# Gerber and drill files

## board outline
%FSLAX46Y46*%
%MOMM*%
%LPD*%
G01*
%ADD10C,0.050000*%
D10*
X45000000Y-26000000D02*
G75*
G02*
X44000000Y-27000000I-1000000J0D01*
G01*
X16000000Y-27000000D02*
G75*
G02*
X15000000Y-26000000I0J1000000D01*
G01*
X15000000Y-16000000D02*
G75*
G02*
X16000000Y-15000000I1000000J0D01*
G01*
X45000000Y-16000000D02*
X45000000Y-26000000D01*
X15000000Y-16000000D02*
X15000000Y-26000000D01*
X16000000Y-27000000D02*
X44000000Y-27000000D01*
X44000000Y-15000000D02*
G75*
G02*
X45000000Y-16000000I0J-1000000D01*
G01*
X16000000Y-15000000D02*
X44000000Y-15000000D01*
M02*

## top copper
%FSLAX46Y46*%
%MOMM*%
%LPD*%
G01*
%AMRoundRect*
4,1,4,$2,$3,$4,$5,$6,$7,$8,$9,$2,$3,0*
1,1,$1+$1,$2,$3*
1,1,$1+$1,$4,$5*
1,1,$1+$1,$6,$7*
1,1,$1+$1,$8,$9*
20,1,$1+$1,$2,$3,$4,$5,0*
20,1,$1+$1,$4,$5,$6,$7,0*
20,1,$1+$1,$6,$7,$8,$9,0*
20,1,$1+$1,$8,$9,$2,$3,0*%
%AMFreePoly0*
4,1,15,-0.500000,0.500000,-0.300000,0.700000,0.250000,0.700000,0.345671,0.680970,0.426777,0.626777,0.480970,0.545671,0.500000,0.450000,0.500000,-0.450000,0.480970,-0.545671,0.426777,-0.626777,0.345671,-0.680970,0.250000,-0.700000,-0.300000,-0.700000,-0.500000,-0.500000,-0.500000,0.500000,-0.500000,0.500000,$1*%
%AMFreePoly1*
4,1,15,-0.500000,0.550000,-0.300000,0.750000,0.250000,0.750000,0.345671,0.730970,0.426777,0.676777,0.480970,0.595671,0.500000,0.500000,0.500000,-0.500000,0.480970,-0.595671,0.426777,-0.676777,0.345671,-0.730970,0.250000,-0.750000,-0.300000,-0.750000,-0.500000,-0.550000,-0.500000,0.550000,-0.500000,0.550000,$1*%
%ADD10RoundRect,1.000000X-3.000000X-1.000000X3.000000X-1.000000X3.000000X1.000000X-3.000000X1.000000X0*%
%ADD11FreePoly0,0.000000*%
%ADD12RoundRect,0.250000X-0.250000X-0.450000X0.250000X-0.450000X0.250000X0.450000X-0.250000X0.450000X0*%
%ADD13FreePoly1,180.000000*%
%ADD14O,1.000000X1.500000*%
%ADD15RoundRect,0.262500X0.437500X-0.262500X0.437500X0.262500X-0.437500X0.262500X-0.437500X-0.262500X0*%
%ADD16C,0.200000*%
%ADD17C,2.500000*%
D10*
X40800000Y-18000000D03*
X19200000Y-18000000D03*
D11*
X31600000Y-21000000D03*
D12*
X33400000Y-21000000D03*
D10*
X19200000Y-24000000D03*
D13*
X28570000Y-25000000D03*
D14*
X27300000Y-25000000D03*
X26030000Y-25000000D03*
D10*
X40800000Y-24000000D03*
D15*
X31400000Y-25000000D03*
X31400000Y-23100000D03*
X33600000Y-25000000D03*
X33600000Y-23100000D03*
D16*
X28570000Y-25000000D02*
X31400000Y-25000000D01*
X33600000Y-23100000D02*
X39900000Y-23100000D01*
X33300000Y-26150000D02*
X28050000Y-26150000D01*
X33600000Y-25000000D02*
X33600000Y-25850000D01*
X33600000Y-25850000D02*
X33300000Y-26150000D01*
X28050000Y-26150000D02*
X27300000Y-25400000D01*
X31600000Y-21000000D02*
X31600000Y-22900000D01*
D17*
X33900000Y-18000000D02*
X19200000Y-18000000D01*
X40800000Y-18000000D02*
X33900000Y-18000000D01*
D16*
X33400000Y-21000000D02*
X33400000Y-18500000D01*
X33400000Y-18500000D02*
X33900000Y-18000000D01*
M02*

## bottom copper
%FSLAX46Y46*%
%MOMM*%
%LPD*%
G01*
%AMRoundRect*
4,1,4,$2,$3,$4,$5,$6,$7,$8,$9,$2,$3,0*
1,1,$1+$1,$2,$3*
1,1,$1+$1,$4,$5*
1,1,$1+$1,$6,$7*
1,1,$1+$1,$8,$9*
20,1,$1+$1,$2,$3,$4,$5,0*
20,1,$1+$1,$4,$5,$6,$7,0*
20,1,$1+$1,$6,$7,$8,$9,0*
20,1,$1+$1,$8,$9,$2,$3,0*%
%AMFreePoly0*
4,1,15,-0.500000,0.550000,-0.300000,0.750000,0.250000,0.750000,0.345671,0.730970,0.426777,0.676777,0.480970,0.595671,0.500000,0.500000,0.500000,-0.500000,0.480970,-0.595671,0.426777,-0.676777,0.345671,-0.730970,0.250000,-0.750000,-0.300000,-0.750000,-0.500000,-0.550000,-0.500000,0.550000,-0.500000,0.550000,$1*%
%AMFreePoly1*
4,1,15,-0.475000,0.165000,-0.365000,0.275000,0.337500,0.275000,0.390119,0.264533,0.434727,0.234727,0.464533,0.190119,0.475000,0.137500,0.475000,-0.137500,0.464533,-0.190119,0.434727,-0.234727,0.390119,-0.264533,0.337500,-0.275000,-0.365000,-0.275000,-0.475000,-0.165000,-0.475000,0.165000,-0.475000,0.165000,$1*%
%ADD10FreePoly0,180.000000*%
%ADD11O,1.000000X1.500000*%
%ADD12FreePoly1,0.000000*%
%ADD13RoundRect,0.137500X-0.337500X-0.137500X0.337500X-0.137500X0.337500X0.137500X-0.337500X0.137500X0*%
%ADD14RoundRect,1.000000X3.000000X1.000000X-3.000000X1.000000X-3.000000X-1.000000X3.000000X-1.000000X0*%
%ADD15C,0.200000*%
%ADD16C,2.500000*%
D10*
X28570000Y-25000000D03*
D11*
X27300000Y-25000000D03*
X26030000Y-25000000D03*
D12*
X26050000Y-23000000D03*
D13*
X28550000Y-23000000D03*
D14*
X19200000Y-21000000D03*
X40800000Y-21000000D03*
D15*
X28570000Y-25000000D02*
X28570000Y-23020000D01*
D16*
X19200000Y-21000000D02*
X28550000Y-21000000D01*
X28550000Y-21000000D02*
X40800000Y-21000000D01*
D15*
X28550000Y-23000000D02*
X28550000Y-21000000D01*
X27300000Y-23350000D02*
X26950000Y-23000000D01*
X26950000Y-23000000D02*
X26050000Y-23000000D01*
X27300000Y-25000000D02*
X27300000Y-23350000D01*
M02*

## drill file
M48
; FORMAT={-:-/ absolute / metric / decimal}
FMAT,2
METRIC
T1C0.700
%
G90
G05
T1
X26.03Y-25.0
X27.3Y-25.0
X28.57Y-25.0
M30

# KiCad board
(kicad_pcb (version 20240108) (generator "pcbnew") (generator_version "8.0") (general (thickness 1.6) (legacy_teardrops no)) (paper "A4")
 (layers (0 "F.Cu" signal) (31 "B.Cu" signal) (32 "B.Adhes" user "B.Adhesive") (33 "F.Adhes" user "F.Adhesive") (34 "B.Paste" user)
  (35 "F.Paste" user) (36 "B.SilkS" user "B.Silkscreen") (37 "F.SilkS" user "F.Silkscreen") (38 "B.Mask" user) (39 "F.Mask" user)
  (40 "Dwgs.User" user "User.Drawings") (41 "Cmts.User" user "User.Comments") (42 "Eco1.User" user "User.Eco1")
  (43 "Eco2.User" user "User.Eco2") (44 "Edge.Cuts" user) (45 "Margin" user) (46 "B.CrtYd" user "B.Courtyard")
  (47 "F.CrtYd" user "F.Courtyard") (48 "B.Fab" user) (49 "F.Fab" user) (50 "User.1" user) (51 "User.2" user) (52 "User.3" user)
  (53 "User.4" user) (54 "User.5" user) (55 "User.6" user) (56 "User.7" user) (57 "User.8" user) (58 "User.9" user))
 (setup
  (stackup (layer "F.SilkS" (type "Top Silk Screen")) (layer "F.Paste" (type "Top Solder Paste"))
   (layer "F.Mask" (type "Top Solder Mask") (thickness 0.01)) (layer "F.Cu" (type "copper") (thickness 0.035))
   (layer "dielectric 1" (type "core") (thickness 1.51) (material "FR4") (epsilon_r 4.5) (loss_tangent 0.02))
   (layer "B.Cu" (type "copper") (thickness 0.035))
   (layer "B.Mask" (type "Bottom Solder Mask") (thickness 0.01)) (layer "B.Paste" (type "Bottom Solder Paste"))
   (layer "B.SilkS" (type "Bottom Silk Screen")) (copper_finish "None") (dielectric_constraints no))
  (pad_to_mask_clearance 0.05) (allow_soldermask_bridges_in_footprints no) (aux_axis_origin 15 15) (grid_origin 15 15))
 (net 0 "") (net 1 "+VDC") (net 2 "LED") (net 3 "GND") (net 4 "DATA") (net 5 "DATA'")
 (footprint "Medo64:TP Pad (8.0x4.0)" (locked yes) (layer "F.Cu") (at 40.8 18)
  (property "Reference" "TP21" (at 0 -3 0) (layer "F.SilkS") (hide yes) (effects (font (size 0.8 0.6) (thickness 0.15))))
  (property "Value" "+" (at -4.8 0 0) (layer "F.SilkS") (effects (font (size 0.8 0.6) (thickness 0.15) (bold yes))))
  (pad "1" smd roundrect (at 0 0) (size 8 4) (layers "F.Cu" "F.Mask") (roundrect_rratio 0.25) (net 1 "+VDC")))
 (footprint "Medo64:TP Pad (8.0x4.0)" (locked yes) (layer "F.Cu") (at 19.2 18)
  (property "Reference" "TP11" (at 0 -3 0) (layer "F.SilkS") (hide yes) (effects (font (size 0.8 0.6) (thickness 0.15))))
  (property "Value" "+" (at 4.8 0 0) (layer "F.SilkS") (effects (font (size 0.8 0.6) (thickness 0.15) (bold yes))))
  (pad "1" smd roundrect (at 0 0) (size 8 4) (layers "F.Cu" "F.Mask") (roundrect_rratio 0.25) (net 1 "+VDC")))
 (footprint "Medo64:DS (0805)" (layer "F.Cu") (at 32.5 21)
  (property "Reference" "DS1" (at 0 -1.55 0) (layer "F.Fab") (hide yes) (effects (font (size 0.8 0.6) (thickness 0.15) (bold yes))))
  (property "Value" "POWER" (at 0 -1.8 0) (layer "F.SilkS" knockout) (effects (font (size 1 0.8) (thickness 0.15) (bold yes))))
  (pad "1" smd roundrect (at -0.9 0) (size 1 1.4) (layers "F.Cu" "F.Paste" "F.Mask") (roundrect_rratio 0.25) (chamfer_ratio 0.2)
   (chamfer top_left bottom_left) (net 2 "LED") (thermal_bridge_angle 45))
  (pad "2" smd roundrect (at 0.9 0) (size 1 1.4) (layers "F.Cu" "F.Paste" "F.Mask") (roundrect_rratio 0.25) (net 1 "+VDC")
   (thermal_bridge_angle 45)))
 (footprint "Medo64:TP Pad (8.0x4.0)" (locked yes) (layer "F.Cu") (at 19.2 24)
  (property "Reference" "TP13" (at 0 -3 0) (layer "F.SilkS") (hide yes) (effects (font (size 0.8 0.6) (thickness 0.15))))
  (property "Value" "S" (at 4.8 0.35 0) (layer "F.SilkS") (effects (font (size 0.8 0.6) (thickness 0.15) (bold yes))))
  (pad "1" smd roundrect (at 0 0) (size 8 4) (layers "F.Cu" "F.Mask") (roundrect_rratio 0.25)))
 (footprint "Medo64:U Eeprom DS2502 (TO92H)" (layer "F.Cu") (at 27.3 25 180)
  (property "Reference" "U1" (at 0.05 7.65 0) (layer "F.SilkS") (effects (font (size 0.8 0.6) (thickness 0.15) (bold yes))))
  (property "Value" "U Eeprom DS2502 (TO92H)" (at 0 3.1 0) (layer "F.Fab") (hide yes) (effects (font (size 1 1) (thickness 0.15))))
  (pad "1" thru_hole roundrect (at -1.27 0 180) (size 1 1.5) (drill 0.7) (layers "*.Cu" "B.Mask") (remove_unused_layers no)
   (roundrect_rratio 0.25) (chamfer_ratio 0.2) (chamfer top_left bottom_left) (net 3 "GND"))
  (pad "2" thru_hole oval (at 0 0 180) (size 1 1.5) (drill 0.7) (layers "*.Cu" "B.Mask") (remove_unused_layers no) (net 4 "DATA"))
  (pad "3" thru_hole oval (at 1.27 0 180) (size 1 1.5) (drill 0.7) (layers "*.Cu" "B.Mask") (remove_unused_layers no)))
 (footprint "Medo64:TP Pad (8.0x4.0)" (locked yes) (layer "F.Cu") (at 40.8 24)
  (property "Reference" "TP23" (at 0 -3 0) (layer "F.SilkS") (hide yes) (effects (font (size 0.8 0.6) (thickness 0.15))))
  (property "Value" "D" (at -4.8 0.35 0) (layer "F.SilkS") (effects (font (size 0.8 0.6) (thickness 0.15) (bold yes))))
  (pad "1" smd roundrect (at 0 0) (size 8 4) (layers "F.Cu" "F.Mask") (roundrect_rratio 0.25) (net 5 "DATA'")))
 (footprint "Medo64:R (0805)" (layer "F.Cu") (at 31.4 24.05 90)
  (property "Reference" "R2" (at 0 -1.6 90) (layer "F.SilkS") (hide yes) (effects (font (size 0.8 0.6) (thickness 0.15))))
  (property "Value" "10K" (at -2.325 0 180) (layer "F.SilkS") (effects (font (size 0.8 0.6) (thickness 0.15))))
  (pad "1" smd roundrect (at -0.95 0 90) (size 1.05 1.4) (layers "F.Cu" "F.Paste" "F.Mask") (roundrect_rratio 0.25) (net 3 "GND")
   (thermal_bridge_angle 45))
  (pad "2" smd roundrect (at 0.95 0 90) (size 1.05 1.4) (layers "F.Cu" "F.Paste" "F.Mask") (roundrect_rratio 0.25) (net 2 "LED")
   (thermal_bridge_angle 45)))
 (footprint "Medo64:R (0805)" (layer "F.Cu") (at 33.6 24.05 90)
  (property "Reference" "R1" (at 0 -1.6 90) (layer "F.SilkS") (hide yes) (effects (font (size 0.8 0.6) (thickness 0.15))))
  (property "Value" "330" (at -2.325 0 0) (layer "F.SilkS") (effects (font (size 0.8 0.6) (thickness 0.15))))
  (pad "1" smd roundrect (at -0.95 0 90) (size 1.05 1.4) (layers "F.Cu" "F.Paste" "F.Mask") (roundrect_rratio 0.25) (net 4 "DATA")
   (thermal_bridge_angle 45))
  (pad "2" smd roundrect (at 0.95 0 90) (size 1.05 1.4) (layers "F.Cu" "F.Paste" "F.Mask") (roundrect_rratio 0.25) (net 5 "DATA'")
   (thermal_bridge_angle 45)))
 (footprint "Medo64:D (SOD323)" (layer "B.Cu") (at 27.3 23)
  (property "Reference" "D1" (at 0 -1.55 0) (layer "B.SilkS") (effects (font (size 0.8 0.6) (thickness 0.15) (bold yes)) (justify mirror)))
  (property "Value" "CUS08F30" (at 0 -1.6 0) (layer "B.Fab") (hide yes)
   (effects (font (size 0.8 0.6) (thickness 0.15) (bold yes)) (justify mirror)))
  (pad "1" smd roundrect (at -1.25 0) (size 0.95 0.55) (layers "B.Cu" "B.Paste" "B.Mask") (roundrect_rratio 0.25) (chamfer_ratio 0.2)
   (chamfer top_left bottom_left) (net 4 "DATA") (thermal_bridge_angle 45))
  (pad "2" smd roundrect (at 1.25 0) (size 0.95 0.55) (layers "B.Cu" "B.Paste" "B.Mask") (roundrect_rratio 0.25) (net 3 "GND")
   (thermal_bridge_angle 45)))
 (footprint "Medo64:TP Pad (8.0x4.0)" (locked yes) (layer "B.Cu") (at 19.2 21 180)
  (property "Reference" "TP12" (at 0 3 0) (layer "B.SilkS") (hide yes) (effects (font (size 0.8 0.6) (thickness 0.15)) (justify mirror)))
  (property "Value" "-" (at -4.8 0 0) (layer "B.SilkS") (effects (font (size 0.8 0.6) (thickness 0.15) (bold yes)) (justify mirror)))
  (pad "1" smd roundrect (at 0 0 180) (size 8 4) (layers "B.Cu" "B.Mask") (roundrect_rratio 0.25) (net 3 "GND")))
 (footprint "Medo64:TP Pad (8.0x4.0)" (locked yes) (layer "B.Cu") (at 40.8 21 180)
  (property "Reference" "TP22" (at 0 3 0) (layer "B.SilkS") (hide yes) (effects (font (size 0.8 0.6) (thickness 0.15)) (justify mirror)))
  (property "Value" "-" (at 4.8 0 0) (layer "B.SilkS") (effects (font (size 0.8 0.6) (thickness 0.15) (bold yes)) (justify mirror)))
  (pad "1" smd roundrect (at 0 0 180) (size 8 4) (layers "B.Cu" "B.Mask") (roundrect_rratio 0.25) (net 3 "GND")))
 (gr_arc (start 45 26) (mid 44.707107 26.707107) (end 44 27) (locked yes) (stroke (width 0.05) (type default)) (layer "Edge.Cuts"))
 (gr_arc (start 16 27) (mid 15.292893 26.707107) (end 15 26) (locked yes) (stroke (width 0.05) (type default)) (layer "Edge.Cuts"))
 (gr_arc (start 15 16) (mid 15.292893 15.292893) (end 16 15) (locked yes) (stroke (width 0.05) (type default)) (layer "Edge.Cuts"))
 (gr_line (start 45 16) (end 45 26) (locked yes) (stroke (width 0.05) (type default)) (layer "Edge.Cuts"))
 (gr_line (start 15 16) (end 15 26) (locked yes) (stroke (width 0.05) (type default)) (layer "Edge.Cuts"))
 (gr_line (start 16 27) (end 44 27) (locked yes) (stroke (width 0.05) (type default)) (layer "Edge.Cuts"))
 (gr_arc (start 44 15) (mid 44.707107 15.292893) (end 45 16) (locked yes) (stroke (width 0.05) (type default)) (layer "Edge.Cuts"))
 (gr_line (start 16 15) (end 44 15) (locked yes) (stroke (width 0.05) (type default)) (layer "Edge.Cuts"))
 (segment (start 28.57 25) (end 31.4 25) (width 0.2) (layer "F.Cu") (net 3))
 (segment (start 28.57 25) (end 28.57 23.02) (width 0.2) (layer "B.Cu") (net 3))
 (segment (start 19.2 21) (end 28.55 21) (width 2.5) (layer "B.Cu") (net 3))
 (segment (start 28.55 21) (end 40.8 21) (width 2.5) (layer "B.Cu") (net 3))
 (segment (start 28.55 23) (end 28.55 21) (width 0.2) (layer "B.Cu") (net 3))
 (segment (start 33.6 23.1) (end 39.9 23.1) (width 0.2) (layer "F.Cu") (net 5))
 (segment (start 33.3 26.15) (end 28.05 26.15) (width 0.2) (layer "F.Cu") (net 4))
 (segment (start 33.6 25) (end 33.6 25.85) (width 0.2) (layer "F.Cu") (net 4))
 (segment (start 33.6 25.85) (end 33.3 26.15) (width 0.2) (layer "F.Cu") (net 4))
 (segment (start 28.05 26.15) (end 27.3 25.4) (width 0.2) (layer "F.Cu") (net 4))
 (segment (start 27.3 23.35) (end 26.95 23) (width 0.2) (layer "B.Cu") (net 4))
 (segment (start 26.95 23) (end 26.05 23) (width 0.2) (layer "B.Cu") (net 4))
 (segment (start 27.3 25) (end 27.3 23.35) (width 0.2) (layer "B.Cu") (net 4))
 (segment (start 31.6 21) (end 31.6 22.9) (width 0.2) (layer "F.Cu") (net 2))
 (segment (start 33.9 18) (end 19.2 18) (width 2.5) (layer "F.Cu") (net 1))
 (segment (start 40.8 18) (end 33.9 18) (width 2.5) (layer "F.Cu") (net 1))
 (segment (start 33.4 21) (end 33.4 18.5) (width 0.2) (layer "F.Cu") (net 1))
 (segment (start 33.4 18.5) (end 33.9 18) (width 0.2) (layer "F.Cu") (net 1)))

